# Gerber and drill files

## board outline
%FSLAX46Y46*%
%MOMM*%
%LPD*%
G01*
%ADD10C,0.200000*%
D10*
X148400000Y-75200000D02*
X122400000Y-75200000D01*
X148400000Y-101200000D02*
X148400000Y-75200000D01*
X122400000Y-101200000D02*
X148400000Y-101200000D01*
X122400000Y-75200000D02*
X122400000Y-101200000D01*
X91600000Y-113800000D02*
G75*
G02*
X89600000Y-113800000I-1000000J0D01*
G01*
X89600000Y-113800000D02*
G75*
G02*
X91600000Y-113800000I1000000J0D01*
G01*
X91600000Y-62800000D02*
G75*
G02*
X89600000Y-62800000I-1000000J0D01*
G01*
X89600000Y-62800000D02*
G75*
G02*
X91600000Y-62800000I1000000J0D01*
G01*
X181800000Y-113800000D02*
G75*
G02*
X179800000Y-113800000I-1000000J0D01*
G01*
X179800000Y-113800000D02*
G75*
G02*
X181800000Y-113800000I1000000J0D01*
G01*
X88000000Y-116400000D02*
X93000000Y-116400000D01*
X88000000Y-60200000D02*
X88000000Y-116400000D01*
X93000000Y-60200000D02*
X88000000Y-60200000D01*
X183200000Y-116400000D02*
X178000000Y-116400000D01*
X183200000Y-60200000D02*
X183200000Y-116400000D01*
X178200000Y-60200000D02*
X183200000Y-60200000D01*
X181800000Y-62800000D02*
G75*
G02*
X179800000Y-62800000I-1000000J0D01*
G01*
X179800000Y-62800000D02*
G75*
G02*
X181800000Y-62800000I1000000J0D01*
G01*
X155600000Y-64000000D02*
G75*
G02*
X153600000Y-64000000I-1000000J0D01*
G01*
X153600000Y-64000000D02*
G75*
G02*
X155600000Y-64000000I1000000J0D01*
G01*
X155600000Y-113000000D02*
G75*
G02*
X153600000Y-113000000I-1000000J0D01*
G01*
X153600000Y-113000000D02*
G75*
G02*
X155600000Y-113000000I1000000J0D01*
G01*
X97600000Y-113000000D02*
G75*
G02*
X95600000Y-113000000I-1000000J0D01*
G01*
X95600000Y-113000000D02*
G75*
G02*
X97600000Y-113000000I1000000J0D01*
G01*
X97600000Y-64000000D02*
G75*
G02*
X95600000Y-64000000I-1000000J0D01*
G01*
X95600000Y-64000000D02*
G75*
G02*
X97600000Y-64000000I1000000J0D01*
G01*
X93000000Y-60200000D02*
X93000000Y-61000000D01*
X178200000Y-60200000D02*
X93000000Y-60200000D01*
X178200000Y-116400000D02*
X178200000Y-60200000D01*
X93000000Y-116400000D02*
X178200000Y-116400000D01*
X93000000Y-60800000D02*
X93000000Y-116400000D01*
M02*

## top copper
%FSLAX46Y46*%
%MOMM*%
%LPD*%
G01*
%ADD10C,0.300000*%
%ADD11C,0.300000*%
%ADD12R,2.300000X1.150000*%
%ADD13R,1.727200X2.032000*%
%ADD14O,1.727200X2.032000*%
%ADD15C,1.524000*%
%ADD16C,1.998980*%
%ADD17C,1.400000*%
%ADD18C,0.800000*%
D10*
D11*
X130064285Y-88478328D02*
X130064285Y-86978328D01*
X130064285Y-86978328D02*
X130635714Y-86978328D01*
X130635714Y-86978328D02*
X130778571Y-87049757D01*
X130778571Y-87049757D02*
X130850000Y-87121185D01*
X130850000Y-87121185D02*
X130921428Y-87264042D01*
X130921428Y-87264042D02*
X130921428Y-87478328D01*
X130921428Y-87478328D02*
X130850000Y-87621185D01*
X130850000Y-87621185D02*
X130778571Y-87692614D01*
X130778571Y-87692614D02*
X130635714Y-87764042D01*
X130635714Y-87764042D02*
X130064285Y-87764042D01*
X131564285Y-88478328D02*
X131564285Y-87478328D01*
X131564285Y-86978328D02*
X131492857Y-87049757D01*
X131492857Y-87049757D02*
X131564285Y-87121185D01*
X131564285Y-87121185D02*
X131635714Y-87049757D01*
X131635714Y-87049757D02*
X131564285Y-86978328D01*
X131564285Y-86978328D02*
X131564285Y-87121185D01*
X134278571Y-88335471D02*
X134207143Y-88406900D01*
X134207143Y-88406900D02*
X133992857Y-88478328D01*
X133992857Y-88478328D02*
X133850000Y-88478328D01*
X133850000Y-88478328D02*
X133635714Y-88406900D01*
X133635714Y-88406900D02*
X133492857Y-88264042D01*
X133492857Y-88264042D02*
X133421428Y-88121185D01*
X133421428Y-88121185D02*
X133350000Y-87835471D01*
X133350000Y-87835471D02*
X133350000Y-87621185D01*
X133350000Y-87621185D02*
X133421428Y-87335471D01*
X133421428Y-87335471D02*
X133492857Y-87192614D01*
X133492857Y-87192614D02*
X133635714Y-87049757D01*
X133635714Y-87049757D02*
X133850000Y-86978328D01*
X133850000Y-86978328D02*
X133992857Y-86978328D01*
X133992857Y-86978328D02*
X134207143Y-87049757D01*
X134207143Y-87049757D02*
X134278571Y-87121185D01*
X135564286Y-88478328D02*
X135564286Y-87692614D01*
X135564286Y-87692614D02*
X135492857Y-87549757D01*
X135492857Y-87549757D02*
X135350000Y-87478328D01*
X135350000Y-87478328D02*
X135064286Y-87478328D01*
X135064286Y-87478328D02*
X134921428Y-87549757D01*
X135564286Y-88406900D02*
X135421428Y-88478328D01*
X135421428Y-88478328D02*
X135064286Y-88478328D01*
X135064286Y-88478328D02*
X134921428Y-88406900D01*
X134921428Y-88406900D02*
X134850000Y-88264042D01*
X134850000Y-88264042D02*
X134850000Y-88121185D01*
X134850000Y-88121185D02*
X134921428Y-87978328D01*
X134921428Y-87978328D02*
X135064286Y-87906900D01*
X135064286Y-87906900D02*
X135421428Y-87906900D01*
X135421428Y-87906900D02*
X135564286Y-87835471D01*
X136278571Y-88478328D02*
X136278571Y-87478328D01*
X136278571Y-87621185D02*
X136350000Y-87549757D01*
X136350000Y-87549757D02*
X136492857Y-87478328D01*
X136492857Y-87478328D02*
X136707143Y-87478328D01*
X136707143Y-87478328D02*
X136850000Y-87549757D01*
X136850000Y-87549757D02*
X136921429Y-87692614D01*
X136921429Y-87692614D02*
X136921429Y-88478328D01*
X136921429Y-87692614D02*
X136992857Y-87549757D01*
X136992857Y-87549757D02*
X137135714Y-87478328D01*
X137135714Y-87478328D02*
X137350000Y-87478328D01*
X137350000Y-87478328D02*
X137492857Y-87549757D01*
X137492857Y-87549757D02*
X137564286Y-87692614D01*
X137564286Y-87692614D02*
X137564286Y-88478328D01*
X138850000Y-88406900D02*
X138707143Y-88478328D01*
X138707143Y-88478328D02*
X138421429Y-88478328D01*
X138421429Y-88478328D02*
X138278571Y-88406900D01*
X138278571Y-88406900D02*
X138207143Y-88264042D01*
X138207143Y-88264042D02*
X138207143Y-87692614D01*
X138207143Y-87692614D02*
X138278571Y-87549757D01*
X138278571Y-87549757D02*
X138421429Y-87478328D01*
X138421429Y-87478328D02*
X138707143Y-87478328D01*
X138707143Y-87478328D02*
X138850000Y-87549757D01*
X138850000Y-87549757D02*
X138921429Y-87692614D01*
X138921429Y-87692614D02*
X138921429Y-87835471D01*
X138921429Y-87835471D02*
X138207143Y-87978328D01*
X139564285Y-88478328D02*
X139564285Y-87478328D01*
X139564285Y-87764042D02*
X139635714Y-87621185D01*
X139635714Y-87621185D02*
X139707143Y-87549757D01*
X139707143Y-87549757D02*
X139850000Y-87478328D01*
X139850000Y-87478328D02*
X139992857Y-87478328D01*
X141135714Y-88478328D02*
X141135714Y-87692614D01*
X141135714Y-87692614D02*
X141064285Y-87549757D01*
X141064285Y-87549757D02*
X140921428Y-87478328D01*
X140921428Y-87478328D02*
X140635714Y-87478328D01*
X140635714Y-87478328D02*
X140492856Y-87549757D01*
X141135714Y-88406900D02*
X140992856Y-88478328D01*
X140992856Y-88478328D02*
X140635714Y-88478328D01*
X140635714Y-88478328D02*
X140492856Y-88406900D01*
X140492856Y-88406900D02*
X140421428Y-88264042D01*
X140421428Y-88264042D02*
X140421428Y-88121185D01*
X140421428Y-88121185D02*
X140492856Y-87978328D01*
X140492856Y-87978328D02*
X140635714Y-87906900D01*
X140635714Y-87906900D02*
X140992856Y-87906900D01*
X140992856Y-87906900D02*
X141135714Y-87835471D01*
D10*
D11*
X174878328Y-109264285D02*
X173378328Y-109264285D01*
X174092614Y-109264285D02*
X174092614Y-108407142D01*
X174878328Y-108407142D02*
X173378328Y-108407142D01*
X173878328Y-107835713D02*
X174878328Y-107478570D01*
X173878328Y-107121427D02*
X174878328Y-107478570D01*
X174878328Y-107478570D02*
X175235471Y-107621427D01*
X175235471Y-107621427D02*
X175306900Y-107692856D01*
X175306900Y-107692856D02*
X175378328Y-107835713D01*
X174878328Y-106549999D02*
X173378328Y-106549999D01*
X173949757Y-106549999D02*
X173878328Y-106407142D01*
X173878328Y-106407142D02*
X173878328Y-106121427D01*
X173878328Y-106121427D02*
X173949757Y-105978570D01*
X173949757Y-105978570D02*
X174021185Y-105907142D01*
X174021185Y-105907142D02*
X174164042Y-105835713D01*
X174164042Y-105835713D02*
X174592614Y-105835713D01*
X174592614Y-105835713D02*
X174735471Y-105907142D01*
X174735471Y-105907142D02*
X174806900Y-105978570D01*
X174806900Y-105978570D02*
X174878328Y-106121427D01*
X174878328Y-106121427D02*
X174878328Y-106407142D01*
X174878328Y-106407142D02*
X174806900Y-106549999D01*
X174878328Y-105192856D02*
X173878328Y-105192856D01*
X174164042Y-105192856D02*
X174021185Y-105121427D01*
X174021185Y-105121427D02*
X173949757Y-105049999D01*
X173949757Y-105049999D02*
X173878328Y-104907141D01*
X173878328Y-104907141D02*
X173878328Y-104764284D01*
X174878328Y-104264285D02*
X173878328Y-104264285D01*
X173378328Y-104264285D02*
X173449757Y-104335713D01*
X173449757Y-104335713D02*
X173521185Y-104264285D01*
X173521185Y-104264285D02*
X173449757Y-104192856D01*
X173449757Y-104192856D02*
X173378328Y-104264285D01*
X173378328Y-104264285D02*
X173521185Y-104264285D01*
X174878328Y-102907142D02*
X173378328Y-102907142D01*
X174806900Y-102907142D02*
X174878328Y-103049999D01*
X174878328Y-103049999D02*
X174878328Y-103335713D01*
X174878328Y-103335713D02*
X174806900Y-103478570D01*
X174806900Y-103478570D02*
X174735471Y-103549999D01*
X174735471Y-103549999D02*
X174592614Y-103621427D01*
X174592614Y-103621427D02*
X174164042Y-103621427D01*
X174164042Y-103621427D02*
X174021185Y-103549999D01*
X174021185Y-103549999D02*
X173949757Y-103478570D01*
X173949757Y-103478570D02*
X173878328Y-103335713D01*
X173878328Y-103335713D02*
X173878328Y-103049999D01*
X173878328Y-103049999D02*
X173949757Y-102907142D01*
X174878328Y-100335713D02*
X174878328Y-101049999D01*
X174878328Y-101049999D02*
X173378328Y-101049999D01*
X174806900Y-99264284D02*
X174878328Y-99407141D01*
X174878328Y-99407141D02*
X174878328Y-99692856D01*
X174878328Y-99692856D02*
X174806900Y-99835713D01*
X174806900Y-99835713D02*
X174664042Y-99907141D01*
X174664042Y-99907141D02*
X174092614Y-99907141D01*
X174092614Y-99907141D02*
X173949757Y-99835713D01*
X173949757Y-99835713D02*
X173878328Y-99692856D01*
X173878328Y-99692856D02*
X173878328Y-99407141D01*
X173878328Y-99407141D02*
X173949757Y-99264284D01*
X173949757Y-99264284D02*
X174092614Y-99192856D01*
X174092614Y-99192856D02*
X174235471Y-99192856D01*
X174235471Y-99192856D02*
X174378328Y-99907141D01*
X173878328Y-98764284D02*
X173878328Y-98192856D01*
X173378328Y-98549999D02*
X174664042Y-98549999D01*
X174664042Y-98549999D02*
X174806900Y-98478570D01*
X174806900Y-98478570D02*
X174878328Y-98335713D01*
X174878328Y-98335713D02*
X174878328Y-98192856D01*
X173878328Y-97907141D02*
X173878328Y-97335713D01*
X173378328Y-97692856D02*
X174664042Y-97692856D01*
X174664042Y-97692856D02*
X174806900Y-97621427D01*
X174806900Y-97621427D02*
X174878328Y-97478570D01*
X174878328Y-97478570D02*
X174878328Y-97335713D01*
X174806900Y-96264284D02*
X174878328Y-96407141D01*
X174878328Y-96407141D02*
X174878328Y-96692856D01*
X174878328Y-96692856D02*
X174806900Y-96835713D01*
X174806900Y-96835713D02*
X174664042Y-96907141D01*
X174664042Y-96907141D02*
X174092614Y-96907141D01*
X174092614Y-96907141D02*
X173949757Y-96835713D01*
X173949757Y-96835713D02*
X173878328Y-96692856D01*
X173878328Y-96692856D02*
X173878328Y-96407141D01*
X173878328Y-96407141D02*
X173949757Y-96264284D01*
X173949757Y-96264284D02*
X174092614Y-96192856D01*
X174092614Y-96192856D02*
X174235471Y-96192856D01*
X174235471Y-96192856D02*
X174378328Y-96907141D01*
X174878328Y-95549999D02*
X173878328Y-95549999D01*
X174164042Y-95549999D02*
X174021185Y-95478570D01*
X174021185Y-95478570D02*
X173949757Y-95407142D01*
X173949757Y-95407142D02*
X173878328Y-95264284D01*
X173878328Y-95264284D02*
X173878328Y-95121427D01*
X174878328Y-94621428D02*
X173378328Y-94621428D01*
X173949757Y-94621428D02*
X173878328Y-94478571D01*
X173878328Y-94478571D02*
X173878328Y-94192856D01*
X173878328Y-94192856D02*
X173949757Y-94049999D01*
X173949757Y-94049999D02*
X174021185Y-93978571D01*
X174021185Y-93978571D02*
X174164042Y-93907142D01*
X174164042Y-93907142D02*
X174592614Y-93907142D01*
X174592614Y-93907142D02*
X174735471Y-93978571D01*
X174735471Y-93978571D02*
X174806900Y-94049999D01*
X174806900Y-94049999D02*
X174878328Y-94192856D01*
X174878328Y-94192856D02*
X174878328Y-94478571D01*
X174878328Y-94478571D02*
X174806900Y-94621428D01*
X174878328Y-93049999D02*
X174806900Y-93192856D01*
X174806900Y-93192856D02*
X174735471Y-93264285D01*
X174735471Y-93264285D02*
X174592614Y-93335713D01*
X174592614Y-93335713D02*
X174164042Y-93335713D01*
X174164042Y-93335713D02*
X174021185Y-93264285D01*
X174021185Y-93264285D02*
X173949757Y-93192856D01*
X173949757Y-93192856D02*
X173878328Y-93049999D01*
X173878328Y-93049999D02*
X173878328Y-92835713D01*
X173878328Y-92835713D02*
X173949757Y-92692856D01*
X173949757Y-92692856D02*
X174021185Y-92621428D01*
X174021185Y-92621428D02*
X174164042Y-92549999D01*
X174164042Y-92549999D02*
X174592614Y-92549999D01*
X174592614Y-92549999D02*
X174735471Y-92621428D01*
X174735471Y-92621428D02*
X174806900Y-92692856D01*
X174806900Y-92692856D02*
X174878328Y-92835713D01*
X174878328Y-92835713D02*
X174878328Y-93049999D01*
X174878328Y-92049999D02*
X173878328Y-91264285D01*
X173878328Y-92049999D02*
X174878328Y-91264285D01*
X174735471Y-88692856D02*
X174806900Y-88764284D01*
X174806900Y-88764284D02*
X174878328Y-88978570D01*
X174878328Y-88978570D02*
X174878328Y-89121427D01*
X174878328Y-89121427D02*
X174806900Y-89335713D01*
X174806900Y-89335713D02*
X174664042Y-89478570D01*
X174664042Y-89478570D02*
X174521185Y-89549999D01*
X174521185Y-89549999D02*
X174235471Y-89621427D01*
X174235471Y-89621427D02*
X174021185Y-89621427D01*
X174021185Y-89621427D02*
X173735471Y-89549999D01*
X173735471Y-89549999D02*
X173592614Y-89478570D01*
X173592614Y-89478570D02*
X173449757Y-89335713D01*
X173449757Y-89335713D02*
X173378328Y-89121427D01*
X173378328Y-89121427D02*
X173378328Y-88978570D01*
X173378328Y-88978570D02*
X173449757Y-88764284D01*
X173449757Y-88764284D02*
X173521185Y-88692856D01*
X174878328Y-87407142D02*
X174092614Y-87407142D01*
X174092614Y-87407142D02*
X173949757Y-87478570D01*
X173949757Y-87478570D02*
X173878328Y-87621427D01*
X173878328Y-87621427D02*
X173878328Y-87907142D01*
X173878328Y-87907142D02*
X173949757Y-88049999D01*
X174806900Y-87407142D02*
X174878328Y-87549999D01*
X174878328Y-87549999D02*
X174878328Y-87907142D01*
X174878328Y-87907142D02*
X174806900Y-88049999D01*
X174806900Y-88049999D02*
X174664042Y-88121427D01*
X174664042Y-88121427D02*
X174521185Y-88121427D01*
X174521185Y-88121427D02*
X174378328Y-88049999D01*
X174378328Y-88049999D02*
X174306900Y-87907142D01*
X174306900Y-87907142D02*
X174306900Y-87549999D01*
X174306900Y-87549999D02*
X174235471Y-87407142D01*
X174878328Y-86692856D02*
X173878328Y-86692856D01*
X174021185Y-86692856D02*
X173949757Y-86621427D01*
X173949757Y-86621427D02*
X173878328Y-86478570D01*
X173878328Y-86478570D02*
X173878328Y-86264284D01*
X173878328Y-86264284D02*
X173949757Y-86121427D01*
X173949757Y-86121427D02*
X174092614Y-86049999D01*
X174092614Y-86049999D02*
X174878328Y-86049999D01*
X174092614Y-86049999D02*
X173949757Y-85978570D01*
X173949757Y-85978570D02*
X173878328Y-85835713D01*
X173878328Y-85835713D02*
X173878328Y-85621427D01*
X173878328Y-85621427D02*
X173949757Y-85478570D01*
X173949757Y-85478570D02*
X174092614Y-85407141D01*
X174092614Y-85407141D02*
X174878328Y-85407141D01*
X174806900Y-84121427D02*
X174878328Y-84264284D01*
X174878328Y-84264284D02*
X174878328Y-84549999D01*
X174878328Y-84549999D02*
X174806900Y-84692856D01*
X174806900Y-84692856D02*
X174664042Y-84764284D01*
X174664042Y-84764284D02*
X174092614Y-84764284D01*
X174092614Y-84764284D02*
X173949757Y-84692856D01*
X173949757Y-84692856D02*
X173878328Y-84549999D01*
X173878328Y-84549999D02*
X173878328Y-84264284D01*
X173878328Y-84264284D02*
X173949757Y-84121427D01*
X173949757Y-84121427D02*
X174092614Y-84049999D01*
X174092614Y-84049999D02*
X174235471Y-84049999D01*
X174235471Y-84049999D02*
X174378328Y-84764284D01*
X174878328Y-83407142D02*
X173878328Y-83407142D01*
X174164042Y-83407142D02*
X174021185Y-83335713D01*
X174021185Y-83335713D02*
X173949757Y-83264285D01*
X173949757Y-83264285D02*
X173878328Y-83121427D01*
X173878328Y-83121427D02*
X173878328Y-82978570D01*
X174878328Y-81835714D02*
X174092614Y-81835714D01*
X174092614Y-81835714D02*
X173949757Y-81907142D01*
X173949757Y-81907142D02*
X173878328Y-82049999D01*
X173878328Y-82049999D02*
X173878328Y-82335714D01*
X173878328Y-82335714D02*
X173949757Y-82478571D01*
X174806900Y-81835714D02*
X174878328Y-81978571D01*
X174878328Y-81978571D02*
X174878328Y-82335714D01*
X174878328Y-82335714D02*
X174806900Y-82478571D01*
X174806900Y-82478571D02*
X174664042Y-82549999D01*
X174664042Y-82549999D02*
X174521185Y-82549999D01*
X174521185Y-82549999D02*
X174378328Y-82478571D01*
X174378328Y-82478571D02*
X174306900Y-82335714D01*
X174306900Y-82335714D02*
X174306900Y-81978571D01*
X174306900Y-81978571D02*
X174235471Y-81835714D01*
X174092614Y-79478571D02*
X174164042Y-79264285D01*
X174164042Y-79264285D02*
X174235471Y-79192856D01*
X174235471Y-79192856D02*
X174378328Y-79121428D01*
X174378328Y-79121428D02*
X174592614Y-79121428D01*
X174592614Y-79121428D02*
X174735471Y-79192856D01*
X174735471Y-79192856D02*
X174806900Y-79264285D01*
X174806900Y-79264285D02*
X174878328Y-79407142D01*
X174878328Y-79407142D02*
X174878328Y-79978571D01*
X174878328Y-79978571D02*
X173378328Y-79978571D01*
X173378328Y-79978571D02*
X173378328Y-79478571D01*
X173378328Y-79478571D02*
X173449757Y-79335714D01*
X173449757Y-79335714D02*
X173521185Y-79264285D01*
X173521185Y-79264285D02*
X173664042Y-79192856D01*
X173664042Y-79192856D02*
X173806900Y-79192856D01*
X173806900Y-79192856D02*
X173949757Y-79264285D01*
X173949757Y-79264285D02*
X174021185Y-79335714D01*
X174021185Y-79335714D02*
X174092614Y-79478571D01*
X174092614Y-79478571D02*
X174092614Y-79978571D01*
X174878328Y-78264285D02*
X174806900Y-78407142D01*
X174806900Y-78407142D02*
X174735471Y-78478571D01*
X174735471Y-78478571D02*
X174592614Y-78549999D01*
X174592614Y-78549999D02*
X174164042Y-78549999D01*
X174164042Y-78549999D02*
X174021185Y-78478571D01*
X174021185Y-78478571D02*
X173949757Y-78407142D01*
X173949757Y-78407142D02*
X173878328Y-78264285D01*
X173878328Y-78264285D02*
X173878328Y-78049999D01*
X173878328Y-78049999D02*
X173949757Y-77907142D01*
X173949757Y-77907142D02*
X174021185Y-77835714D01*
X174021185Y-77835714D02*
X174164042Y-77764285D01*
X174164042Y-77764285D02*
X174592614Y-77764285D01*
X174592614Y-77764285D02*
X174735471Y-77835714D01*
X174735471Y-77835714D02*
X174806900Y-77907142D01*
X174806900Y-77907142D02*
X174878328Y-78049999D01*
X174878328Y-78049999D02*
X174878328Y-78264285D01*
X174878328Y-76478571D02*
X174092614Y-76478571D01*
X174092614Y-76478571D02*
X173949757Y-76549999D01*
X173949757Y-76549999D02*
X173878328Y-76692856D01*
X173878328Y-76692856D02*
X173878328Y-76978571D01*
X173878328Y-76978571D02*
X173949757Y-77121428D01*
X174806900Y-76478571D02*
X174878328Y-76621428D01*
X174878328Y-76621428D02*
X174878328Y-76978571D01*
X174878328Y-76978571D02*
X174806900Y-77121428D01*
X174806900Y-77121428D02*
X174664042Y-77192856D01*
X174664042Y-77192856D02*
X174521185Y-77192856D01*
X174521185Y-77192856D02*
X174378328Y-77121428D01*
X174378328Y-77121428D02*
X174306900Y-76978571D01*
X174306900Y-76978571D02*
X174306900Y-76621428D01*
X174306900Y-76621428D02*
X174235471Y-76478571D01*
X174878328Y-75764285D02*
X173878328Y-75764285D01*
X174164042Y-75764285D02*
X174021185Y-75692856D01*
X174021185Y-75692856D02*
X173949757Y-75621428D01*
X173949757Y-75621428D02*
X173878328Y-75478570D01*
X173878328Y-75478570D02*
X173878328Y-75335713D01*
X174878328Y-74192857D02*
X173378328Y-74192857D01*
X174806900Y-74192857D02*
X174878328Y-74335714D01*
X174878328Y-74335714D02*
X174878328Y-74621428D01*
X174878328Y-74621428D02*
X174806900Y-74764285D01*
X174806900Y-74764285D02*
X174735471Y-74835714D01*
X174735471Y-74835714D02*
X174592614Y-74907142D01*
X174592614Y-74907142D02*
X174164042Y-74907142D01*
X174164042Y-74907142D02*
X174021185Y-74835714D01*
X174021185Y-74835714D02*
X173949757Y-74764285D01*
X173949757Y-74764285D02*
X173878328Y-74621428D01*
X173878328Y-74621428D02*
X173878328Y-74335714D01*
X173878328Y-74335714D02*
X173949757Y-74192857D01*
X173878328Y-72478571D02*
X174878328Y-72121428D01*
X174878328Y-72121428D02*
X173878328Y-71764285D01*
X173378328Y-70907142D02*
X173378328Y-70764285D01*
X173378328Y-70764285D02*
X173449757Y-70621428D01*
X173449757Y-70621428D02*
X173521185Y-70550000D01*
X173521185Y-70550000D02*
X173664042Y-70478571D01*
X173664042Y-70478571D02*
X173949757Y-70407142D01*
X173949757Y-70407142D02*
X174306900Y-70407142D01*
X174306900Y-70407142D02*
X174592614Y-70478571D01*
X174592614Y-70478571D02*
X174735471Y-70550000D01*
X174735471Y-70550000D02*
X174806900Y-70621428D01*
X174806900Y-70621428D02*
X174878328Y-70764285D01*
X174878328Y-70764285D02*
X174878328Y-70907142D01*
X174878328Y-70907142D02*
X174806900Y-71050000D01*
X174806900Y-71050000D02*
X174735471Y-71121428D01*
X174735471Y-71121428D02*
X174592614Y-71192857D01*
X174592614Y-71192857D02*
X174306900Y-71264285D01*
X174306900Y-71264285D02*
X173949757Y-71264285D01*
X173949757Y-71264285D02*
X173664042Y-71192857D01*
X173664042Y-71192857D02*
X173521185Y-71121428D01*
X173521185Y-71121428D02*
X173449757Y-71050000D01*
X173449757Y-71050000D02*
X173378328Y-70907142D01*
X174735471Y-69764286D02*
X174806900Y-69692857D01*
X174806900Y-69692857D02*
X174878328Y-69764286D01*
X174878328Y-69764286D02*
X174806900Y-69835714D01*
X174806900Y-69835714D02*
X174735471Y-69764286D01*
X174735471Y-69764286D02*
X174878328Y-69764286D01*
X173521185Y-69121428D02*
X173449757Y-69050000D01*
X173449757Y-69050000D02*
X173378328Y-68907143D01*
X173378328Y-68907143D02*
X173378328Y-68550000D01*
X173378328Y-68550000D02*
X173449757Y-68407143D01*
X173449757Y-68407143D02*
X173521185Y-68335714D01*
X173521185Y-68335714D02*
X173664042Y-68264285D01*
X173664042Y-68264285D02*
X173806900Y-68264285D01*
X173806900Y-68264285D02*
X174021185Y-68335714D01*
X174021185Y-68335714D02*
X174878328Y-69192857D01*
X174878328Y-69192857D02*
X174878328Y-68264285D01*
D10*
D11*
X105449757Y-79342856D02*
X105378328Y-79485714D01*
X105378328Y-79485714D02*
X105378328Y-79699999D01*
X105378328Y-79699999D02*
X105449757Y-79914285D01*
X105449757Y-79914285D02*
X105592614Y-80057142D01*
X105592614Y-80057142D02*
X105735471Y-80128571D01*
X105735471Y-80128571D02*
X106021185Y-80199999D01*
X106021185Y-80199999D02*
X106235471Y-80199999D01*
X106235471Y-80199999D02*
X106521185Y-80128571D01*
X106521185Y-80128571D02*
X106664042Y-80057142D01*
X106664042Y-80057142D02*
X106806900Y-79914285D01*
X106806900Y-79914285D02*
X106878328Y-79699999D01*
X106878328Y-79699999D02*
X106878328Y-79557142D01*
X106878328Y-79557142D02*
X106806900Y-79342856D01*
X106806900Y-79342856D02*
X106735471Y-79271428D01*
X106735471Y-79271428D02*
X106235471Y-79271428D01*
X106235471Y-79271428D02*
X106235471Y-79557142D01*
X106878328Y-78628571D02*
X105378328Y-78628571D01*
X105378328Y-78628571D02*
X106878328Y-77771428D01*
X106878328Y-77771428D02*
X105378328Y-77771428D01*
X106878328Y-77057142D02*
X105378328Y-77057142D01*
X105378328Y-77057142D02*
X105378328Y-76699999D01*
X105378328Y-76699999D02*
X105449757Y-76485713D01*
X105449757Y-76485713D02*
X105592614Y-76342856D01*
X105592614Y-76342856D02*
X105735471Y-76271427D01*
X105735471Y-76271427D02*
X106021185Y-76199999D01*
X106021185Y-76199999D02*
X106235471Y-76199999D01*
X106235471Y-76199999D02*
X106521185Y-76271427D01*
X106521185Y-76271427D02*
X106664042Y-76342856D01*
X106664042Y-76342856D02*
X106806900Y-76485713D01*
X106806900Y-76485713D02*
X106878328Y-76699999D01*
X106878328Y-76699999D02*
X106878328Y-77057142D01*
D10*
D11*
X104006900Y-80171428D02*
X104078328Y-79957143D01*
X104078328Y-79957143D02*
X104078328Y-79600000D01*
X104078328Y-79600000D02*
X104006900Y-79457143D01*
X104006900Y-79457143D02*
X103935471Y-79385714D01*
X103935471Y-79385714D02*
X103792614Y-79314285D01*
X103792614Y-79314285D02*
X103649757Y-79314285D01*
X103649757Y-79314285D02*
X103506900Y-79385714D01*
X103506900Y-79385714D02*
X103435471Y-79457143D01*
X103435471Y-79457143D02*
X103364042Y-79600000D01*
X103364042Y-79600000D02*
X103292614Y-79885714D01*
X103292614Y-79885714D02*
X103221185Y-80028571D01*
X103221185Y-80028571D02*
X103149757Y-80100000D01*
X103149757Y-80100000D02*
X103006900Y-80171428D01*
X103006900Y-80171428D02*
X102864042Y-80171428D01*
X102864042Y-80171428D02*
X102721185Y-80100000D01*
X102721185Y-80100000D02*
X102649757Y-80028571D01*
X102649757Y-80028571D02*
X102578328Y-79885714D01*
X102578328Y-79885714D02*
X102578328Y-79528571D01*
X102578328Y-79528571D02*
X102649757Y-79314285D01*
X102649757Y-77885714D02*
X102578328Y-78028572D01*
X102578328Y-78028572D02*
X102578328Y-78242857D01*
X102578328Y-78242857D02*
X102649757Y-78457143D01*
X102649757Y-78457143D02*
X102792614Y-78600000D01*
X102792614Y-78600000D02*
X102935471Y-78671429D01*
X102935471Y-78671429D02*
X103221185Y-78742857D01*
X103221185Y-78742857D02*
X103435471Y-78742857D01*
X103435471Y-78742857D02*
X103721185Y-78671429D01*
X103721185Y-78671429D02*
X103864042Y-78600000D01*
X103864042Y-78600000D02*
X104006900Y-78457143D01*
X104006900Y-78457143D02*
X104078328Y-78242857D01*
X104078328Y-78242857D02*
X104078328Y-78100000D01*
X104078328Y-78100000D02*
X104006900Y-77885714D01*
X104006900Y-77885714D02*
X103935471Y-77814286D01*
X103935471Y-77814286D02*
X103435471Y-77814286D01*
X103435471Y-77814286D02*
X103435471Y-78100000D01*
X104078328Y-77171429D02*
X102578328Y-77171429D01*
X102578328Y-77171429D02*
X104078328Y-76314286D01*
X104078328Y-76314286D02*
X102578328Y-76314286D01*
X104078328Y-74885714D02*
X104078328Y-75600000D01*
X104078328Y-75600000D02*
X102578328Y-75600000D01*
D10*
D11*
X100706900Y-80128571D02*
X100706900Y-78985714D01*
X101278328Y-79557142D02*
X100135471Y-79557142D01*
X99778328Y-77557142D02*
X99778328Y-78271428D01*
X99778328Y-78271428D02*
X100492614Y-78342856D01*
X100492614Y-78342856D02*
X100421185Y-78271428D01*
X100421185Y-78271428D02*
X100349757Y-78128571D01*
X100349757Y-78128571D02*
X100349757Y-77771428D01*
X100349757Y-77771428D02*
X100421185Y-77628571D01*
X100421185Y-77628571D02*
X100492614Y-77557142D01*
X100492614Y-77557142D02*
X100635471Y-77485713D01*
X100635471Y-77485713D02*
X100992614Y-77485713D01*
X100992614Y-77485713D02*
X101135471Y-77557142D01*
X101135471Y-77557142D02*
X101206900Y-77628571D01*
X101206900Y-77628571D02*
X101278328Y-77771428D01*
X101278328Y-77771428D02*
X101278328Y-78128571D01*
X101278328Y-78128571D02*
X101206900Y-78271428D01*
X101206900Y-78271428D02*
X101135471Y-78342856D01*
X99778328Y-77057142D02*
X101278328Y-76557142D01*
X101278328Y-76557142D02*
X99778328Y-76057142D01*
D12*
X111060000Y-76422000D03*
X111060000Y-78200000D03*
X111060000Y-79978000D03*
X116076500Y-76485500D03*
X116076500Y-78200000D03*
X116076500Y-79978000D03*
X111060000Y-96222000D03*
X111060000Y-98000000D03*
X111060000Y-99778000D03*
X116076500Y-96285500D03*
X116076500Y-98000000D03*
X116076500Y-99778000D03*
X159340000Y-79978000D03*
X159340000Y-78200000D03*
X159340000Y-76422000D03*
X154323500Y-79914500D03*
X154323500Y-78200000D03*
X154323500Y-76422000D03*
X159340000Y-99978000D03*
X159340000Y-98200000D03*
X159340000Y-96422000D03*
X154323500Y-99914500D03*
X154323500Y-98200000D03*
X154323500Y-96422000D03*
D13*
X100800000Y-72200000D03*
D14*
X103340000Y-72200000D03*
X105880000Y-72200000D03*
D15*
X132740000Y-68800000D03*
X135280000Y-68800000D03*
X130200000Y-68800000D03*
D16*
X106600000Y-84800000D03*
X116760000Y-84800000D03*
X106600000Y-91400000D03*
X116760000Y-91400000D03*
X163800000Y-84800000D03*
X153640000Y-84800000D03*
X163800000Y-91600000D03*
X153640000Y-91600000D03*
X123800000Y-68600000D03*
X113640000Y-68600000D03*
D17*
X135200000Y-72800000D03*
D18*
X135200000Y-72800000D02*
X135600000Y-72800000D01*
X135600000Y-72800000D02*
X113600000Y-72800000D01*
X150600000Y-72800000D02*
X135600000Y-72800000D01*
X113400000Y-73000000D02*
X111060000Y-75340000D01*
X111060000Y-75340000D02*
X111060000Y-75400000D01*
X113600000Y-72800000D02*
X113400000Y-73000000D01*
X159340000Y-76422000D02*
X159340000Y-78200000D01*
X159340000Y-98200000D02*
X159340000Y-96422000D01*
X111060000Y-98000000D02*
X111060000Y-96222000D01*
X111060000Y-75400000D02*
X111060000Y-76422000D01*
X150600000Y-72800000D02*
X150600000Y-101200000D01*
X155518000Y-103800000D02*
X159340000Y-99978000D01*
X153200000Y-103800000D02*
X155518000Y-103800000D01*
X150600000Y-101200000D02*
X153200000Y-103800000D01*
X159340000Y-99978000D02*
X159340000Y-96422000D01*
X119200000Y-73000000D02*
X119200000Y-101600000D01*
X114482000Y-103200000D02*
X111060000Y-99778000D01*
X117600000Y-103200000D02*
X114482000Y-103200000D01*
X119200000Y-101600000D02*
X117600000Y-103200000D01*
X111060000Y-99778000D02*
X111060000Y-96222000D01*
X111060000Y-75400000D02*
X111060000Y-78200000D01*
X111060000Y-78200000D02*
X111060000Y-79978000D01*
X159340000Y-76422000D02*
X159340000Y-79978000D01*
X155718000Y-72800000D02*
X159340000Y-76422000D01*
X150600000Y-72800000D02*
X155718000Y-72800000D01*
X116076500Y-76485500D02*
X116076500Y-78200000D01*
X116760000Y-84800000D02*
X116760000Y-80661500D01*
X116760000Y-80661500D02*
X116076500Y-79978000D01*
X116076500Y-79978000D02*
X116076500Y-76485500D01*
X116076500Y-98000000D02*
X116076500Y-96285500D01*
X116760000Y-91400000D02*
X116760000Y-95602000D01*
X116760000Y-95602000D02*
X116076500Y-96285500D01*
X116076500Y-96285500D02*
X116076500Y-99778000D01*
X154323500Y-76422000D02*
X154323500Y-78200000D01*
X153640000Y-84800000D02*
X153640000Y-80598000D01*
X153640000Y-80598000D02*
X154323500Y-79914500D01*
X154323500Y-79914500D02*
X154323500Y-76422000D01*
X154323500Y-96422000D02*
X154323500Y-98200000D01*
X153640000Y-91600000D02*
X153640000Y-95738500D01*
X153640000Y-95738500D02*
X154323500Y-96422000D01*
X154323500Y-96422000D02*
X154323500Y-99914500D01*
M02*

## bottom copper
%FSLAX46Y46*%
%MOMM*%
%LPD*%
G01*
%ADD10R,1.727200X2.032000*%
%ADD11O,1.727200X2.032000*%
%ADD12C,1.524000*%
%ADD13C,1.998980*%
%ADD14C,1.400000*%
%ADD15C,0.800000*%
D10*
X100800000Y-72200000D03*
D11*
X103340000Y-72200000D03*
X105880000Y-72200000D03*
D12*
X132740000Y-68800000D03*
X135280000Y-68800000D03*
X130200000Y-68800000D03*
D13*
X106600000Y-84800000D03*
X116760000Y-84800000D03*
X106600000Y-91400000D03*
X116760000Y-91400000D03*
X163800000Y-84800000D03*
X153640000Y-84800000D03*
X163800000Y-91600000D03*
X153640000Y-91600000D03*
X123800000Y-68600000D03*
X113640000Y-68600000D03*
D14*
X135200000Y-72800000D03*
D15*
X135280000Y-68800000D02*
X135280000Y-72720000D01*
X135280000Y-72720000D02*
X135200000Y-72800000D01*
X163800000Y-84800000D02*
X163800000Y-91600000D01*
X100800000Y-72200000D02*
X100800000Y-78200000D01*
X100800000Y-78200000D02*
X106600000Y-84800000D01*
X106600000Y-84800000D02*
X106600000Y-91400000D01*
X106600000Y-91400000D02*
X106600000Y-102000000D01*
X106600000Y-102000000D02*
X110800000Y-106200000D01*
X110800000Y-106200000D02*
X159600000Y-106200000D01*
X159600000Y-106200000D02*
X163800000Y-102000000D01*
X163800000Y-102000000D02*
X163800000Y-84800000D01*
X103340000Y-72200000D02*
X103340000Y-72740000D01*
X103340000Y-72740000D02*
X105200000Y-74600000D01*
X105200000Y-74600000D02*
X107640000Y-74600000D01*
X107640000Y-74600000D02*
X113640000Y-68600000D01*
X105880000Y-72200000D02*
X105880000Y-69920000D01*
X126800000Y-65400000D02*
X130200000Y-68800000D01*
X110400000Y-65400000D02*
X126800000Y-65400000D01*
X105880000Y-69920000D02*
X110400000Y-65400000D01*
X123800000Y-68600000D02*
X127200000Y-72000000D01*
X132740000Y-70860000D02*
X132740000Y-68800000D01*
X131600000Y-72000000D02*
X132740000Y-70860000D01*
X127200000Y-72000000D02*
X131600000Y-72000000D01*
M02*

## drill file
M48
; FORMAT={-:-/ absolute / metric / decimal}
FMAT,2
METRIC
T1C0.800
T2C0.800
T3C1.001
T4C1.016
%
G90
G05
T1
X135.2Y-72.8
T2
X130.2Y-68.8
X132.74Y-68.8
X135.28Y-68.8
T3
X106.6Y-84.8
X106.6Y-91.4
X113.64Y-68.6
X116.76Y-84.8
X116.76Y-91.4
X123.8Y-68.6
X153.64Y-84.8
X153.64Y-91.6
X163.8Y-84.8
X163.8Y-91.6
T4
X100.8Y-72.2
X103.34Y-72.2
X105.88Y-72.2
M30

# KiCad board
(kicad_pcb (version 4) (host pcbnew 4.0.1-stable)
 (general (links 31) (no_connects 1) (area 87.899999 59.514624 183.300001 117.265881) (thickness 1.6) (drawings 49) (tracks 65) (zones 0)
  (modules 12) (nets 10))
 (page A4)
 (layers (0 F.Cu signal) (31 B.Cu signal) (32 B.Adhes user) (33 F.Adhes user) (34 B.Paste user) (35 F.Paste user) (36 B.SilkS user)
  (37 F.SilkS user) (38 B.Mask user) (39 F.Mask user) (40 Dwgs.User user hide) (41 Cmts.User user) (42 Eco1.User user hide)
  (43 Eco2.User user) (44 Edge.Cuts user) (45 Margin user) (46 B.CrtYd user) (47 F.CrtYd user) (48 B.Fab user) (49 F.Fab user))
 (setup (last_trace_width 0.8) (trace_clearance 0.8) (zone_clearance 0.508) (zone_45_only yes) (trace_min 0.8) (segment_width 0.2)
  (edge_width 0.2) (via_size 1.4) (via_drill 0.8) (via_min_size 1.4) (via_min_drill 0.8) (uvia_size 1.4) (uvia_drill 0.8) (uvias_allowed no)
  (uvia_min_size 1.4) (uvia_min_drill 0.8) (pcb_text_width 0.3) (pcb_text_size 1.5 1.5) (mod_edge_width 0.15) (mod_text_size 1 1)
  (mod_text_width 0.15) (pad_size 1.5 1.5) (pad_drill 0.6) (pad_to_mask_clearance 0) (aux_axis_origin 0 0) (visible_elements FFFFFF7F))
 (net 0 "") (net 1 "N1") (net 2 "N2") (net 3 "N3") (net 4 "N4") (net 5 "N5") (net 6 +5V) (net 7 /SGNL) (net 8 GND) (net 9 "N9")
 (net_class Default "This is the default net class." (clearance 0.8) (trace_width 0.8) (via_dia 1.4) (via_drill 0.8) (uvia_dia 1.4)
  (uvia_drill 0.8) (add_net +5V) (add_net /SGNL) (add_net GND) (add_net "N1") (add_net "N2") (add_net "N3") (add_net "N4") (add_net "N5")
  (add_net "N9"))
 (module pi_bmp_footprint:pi (layer F.Cu) (at 135.4 88.2)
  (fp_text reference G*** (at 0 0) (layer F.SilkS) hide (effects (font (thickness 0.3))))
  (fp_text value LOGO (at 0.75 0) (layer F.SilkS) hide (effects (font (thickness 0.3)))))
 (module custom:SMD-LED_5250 (layer F.Cu) (at 113.6 78.2)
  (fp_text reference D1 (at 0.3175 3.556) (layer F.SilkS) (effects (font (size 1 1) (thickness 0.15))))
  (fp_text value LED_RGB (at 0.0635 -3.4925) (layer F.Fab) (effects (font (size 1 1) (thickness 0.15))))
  (pad 1 smd rect (at -2.54 -1.778) (size 2.3 1.15) (layers F.Cu F.Paste F.Mask) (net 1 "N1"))
  (pad 2 smd rect (at -2.54 0) (size 2.3 1.15) (layers F.Cu F.Paste F.Mask) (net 1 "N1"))
  (pad 3 smd rect (at -2.54 1.778) (size 2.3 1.15) (layers F.Cu F.Paste F.Mask) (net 1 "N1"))
  (pad 4 smd rect (at 2.4765 -1.7145) (size 2.3 1.15) (layers F.Cu F.Paste F.Mask) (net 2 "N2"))
  (pad 5 smd rect (at 2.4765 0) (size 2.3 1.15) (layers F.Cu F.Paste F.Mask) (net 2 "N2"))
  (pad 6 smd rect (at 2.4765 1.778) (size 2.3 1.15) (layers F.Cu F.Paste F.Mask) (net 2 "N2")))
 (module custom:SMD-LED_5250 (layer F.Cu) (at 113.6 98)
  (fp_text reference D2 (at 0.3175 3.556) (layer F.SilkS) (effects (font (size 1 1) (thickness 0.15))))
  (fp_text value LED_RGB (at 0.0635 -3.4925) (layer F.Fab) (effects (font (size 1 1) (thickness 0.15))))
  (pad 1 smd rect (at -2.54 -1.778) (size 2.3 1.15) (layers F.Cu F.Paste F.Mask) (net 1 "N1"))
  (pad 2 smd rect (at -2.54 0) (size 2.3 1.15) (layers F.Cu F.Paste F.Mask) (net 1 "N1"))
  (pad 3 smd rect (at -2.54 1.778) (size 2.3 1.15) (layers F.Cu F.Paste F.Mask) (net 1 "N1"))
  (pad 4 smd rect (at 2.4765 -1.7145) (size 2.3 1.15) (layers F.Cu F.Paste F.Mask) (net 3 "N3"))
  (pad 5 smd rect (at 2.4765 0) (size 2.3 1.15) (layers F.Cu F.Paste F.Mask) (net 3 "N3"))
  (pad 6 smd rect (at 2.4765 1.778) (size 2.3 1.15) (layers F.Cu F.Paste F.Mask) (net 3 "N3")))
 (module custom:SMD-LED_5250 (layer F.Cu) (at 156.8 78.2 180)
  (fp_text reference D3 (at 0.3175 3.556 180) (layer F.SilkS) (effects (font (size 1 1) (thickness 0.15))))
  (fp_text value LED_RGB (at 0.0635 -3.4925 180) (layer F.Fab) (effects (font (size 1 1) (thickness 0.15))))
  (pad 1 smd rect (at -2.54 -1.778 180) (size 2.3 1.15) (layers F.Cu F.Paste F.Mask) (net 1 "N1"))
  (pad 2 smd rect (at -2.54 0 180) (size 2.3 1.15) (layers F.Cu F.Paste F.Mask) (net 1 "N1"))
  (pad 3 smd rect (at -2.54 1.778 180) (size 2.3 1.15) (layers F.Cu F.Paste F.Mask) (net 1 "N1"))
  (pad 4 smd rect (at 2.4765 -1.7145 180) (size 2.3 1.15) (layers F.Cu F.Paste F.Mask) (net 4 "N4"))
  (pad 5 smd rect (at 2.4765 0 180) (size 2.3 1.15) (layers F.Cu F.Paste F.Mask) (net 4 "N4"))
  (pad 6 smd rect (at 2.4765 1.778 180) (size 2.3 1.15) (layers F.Cu F.Paste F.Mask) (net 4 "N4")))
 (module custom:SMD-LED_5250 (layer F.Cu) (at 156.8 98.2 180)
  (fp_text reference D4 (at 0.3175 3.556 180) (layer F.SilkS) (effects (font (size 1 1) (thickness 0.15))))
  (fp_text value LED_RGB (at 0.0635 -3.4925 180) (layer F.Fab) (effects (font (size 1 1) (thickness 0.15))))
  (pad 1 smd rect (at -2.54 -1.778 180) (size 2.3 1.15) (layers F.Cu F.Paste F.Mask) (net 1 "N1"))
  (pad 2 smd rect (at -2.54 0 180) (size 2.3 1.15) (layers F.Cu F.Paste F.Mask) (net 1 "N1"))
  (pad 3 smd rect (at -2.54 1.778 180) (size 2.3 1.15) (layers F.Cu F.Paste F.Mask) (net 1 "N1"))
  (pad 4 smd rect (at 2.4765 -1.7145 180) (size 2.3 1.15) (layers F.Cu F.Paste F.Mask) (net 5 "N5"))
  (pad 5 smd rect (at 2.4765 0 180) (size 2.3 1.15) (layers F.Cu F.Paste F.Mask) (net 5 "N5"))
  (pad 6 smd rect (at 2.4765 1.778 180) (size 2.3 1.15) (layers F.Cu F.Paste F.Mask) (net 5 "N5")))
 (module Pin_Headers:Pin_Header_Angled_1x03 (layer F.Cu) (at 100.8 72.2 90)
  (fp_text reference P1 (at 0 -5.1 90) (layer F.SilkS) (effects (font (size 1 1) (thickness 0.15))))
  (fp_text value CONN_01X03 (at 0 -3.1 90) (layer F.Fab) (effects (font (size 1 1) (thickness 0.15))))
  (pad 1 thru_hole rect (at 0 0 90) (size 2.032 1.7272) (drill 1.016) (layers *.Cu *.Mask F.SilkS) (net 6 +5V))
  (pad 2 thru_hole oval (at 0 2.54 90) (size 2.032 1.7272) (drill 1.016) (layers *.Cu *.Mask F.SilkS) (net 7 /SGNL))
  (pad 3 thru_hole oval (at 0 5.08 90) (size 2.032 1.7272) (drill 1.016) (layers *.Cu *.Mask F.SilkS) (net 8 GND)))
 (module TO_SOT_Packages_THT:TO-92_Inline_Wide (layer F.Cu) (at 130.2 68.8)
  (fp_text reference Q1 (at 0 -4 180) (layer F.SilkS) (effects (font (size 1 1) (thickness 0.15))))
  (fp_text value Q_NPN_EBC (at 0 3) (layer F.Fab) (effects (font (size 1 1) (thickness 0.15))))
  (pad 2 thru_hole circle (at 2.54 0 90) (size 1.524 1.524) (drill 0.8) (layers *.Cu *.Mask F.SilkS) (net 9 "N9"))
  (pad 3 thru_hole circle (at 5.08 0 90) (size 1.524 1.524) (drill 0.8) (layers *.Cu *.Mask F.SilkS) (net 1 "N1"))
  (pad 1 thru_hole circle (at 0 0 90) (size 1.524 1.524) (drill 0.8) (layers *.Cu *.Mask F.SilkS) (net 8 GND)))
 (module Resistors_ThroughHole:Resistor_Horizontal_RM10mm (layer F.Cu) (at 106.6 84.8)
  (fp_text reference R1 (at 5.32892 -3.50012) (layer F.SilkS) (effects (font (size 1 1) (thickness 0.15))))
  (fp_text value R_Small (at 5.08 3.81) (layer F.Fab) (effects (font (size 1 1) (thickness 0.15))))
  (pad 1 thru_hole circle (at 0 0) (size 1.99898 1.99898) (drill 1.00076) (layers *.Cu *.SilkS *.Mask) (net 6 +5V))
  (pad 2 thru_hole circle (at 10.16 0) (size 1.99898 1.99898) (drill 1.00076) (layers *.Cu *.SilkS *.Mask) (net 2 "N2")))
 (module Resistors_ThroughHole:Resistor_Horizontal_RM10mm (layer F.Cu) (at 106.6 91.4)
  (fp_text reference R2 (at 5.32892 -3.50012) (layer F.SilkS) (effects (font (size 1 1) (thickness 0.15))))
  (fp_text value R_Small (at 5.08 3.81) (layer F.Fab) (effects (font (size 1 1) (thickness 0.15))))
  (pad 1 thru_hole circle (at 0 0) (size 1.99898 1.99898) (drill 1.00076) (layers *.Cu *.SilkS *.Mask) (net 6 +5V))
  (pad 2 thru_hole circle (at 10.16 0) (size 1.99898 1.99898) (drill 1.00076) (layers *.Cu *.SilkS *.Mask) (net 3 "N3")))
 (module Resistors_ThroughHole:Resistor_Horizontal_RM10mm (layer F.Cu) (at 163.8 84.8 180)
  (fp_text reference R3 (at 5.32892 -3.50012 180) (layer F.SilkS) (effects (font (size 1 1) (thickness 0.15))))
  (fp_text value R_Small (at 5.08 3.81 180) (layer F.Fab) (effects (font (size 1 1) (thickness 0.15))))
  (pad 1 thru_hole circle (at 0 0 180) (size 1.99898 1.99898) (drill 1.00076) (layers *.Cu *.SilkS *.Mask) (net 6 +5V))
  (pad 2 thru_hole circle (at 10.16 0 180) (size 1.99898 1.99898) (drill 1.00076) (layers *.Cu *.SilkS *.Mask) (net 4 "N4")))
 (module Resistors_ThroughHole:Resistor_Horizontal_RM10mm (layer F.Cu) (at 163.8 91.6 180)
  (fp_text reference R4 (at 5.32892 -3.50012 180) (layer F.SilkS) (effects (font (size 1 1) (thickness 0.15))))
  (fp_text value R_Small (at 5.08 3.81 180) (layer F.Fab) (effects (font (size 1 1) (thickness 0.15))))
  (pad 1 thru_hole circle (at 0 0 180) (size 1.99898 1.99898) (drill 1.00076) (layers *.Cu *.SilkS *.Mask) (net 6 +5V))
  (pad 2 thru_hole circle (at 10.16 0 180) (size 1.99898 1.99898) (drill 1.00076) (layers *.Cu *.SilkS *.Mask) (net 5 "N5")))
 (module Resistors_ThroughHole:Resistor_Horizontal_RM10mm (layer F.Cu) (at 123.8 68.6 180)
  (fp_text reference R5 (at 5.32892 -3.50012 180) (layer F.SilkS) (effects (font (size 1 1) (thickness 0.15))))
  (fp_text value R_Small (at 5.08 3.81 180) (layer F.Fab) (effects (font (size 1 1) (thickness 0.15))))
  (pad 1 thru_hole circle (at 0 0 180) (size 1.99898 1.99898) (drill 1.00076) (layers *.Cu *.SilkS *.Mask) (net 9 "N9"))
  (pad 2 thru_hole circle (at 10.16 0 180) (size 1.99898 1.99898) (drill 1.00076) (layers *.Cu *.SilkS *.Mask) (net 7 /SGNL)))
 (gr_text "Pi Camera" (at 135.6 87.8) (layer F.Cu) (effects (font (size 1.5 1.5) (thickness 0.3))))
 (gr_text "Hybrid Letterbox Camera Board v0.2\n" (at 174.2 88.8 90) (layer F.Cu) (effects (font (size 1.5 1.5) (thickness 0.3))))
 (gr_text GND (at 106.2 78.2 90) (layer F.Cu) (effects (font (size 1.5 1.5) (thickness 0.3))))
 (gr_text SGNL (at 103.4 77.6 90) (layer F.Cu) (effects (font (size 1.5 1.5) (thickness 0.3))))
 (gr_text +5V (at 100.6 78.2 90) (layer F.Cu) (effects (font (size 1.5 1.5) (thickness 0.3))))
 (gr_line (start 148.4 75.2) (end 122.4 75.2) (angle 90) (layer Edge.Cuts) (width 0.2))
 (gr_line (start 148.4 101.2) (end 148.4 75.2) (angle 90) (layer Edge.Cuts) (width 0.2))
 (gr_line (start 122.4 101.2) (end 148.4 101.2) (angle 90) (layer Edge.Cuts) (width 0.2))
 (gr_line (start 122.4 75.2) (end 122.4 101.2) (angle 90) (layer Edge.Cuts) (width 0.2))
 (gr_circle (center 90.6 113.8) (end 91.4 114.4) (layer Edge.Cuts) (width 0.2))
 (gr_circle (center 90.6 62.8) (end 91.4 63.4) (layer Edge.Cuts) (width 0.2))
 (gr_circle (center 180.8 113.8) (end 181.6 114.4) (layer Edge.Cuts) (width 0.2))
 (gr_line (start 88 116.4) (end 93 116.4) (angle 90) (layer Edge.Cuts) (width 0.2))
 (gr_line (start 88 60.2) (end 88 116.4) (angle 90) (layer Edge.Cuts) (width 0.2))
 (gr_line (start 93 60.2) (end 88 60.2) (angle 90) (layer Edge.Cuts) (width 0.2))
 (gr_line (start 183.2 116.4) (end 178 116.4) (angle 90) (layer Edge.Cuts) (width 0.2))
 (gr_line (start 183.2 60.2) (end 183.2 116.4) (angle 90) (layer Edge.Cuts) (width 0.2))
 (gr_line (start 178.2 60.2) (end 183.2 60.2) (angle 90) (layer Edge.Cuts) (width 0.2))
 (gr_circle (center 180.8 62.8) (end 181.6 63.4) (layer Edge.Cuts) (width 0.2))
 (gr_circle (center 154.6 64) (end 155.4 64.6) (layer Edge.Cuts) (width 0.2))
 (gr_circle (center 154.6 113) (end 155.4 113.6) (layer Edge.Cuts) (width 0.2))
 (gr_circle (center 96.6 113) (end 97.4 113.6) (layer Edge.Cuts) (width 0.2))
 (gr_circle (center 96.6 64) (end 97.4 64.6) (layer Edge.Cuts) (width 0.2))
 (gr_line (start 93 60.2) (end 93 61) (angle 90) (layer Edge.Cuts) (width 0.2))
 (gr_line (start 178.2 60.2) (end 93 60.2) (angle 90) (layer Edge.Cuts) (width 0.2))
 (gr_line (start 178.2 116.4) (end 178.2 60.2) (angle 90) (layer Edge.Cuts) (width 0.2))
 (gr_line (start 93 116.4) (end 178.2 116.4) (angle 90) (layer Edge.Cuts) (width 0.2))
 (gr_line (start 93 60.8) (end 93 116.4) (angle 90) (layer Edge.Cuts) (width 0.2))
 (segment (start 135.28 68.8) (end 135.28 72.72) (width 0.8) (layer B.Cu) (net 1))
 (segment (start 135.2 72.8) (end 135.6 72.8) (width 0.8) (layer F.Cu) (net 1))
 (via (at 135.2 72.8) (size 1.4) (drill 0.8) (layers F.Cu B.Cu) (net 1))
 (segment (start 135.28 72.72) (end 135.2 72.8) (width 0.8) (layer B.Cu) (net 1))
 (segment (start 135.6 72.8) (end 113.6 72.8) (width 0.8) (layer F.Cu) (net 1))
 (segment (start 150.6 72.8) (end 135.6 72.8) (width 0.8) (layer F.Cu) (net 1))
 (segment (start 113.4 73) (end 111.06 75.34) (width 0.8) (layer F.Cu) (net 1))
 (segment (start 111.06 75.34) (end 111.06 75.4) (width 0.8) (layer F.Cu) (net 1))
 (segment (start 113.6 72.8) (end 113.4 73) (width 0.8) (layer F.Cu) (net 1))
 (segment (start 159.34 76.422) (end 159.34 78.2) (width 0.8) (layer F.Cu) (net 1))
 (segment (start 159.34 98.2) (end 159.34 96.422) (width 0.8) (layer F.Cu) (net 1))
 (segment (start 111.06 98) (end 111.06 96.222) (width 0.8) (layer F.Cu) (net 1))
 (segment (start 111.06 75.4) (end 111.06 76.422) (width 0.8) (layer F.Cu) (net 1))
 (segment (start 150.6 72.8) (end 150.6 101.2) (width 0.8) (layer F.Cu) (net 1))
 (segment (start 155.518 103.8) (end 159.34 99.978) (width 0.8) (layer F.Cu) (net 1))
 (segment (start 153.2 103.8) (end 155.518 103.8) (width 0.8) (layer F.Cu) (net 1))
 (segment (start 150.6 101.2) (end 153.2 103.8) (width 0.8) (layer F.Cu) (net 1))
 (segment (start 159.34 99.978) (end 159.34 96.422) (width 0.8) (layer F.Cu) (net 1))
 (segment (start 119.2 73) (end 119.2 101.6) (width 0.8) (layer F.Cu) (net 1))
 (segment (start 114.482 103.2) (end 111.06 99.778) (width 0.8) (layer F.Cu) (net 1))
 (segment (start 117.6 103.2) (end 114.482 103.2) (width 0.8) (layer F.Cu) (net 1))
 (segment (start 119.2 101.6) (end 117.6 103.2) (width 0.8) (layer F.Cu) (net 1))
 (segment (start 111.06 99.778) (end 111.06 96.222) (width 0.8) (layer F.Cu) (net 1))
 (segment (start 111.06 75.4) (end 111.06 78.2) (width 0.8) (layer F.Cu) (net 1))
 (segment (start 111.06 78.2) (end 111.06 79.978) (width 0.8) (layer F.Cu) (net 1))
 (segment (start 159.34 76.422) (end 159.34 79.978) (width 0.8) (layer F.Cu) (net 1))
 (segment (start 155.718 72.8) (end 159.34 76.422) (width 0.8) (layer F.Cu) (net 1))
 (segment (start 150.6 72.8) (end 155.718 72.8) (width 0.8) (layer F.Cu) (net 1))
 (segment (start 116.0765 76.4855) (end 116.0765 78.2) (width 0.8) (layer F.Cu) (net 2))
 (segment (start 116.76 84.8) (end 116.76 80.6615) (width 0.8) (layer F.Cu) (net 2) (status 10))
 (segment (start 116.76 80.6615) (end 116.0765 79.978) (width 0.8) (layer F.Cu) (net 2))
 (segment (start 116.0765 79.978) (end 116.0765 76.4855) (width 0.8) (layer F.Cu) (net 2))
 (segment (start 116.0765 98) (end 116.0765 96.2855) (width 0.8) (layer F.Cu) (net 3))
 (segment (start 116.76 91.4) (end 116.76 95.602) (width 0.8) (layer F.Cu) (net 3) (status 10))
 (segment (start 116.76 95.602) (end 116.0765 96.2855) (width 0.8) (layer F.Cu) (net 3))
 (segment (start 116.0765 96.2855) (end 116.0765 99.778) (width 0.8) (layer F.Cu) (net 3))
 (segment (start 154.3235 76.422) (end 154.3235 78.2) (width 0.8) (layer F.Cu) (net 4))
 (segment (start 153.64 84.8) (end 153.64 80.598) (width 0.8) (layer F.Cu) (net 4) (status 10))
 (segment (start 153.64 80.598) (end 154.3235 79.9145) (width 0.8) (layer F.Cu) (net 4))
 (segment (start 154.3235 79.9145) (end 154.3235 76.422) (width 0.8) (layer F.Cu) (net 4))
 (segment (start 154.3235 96.422) (end 154.3235 98.2) (width 0.8) (layer F.Cu) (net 5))
 (segment (start 153.64 91.6) (end 153.64 95.7385) (width 0.8) (layer F.Cu) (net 5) (status 10))
 (segment (start 153.64 95.7385) (end 154.3235 96.422) (width 0.8) (layer F.Cu) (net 5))
 (segment (start 154.3235 96.422) (end 154.3235 99.9145) (width 0.8) (layer F.Cu) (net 5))
 (segment (start 163.8 84.8) (end 163.8 91.6) (width 0.8) (layer B.Cu) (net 6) (status 20))
 (segment (start 100.8 72.2) (end 100.8 78.2) (width 0.8) (layer B.Cu) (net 6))
 (segment (start 100.8 78.2) (end 106.6 84.8) (width 0.8) (layer B.Cu) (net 6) (status 20))
 (segment (start 106.6 84.8) (end 106.6 91.4) (width 0.8) (layer B.Cu) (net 6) (status 10))
 (segment (start 106.6 91.4) (end 106.6 102) (width 0.8) (layer B.Cu) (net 6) (status 10))
 (segment (start 106.6 102) (end 110.8 106.2) (width 0.8) (layer B.Cu) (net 6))
 (segment (start 110.8 106.2) (end 159.6 106.2) (width 0.8) (layer B.Cu) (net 6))
 (segment (start 159.6 106.2) (end 163.8 102) (width 0.8) (layer B.Cu) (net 6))
 (segment (start 163.8 102) (end 163.8 84.8) (width 0.8) (layer B.Cu) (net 6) (status 20))
 (segment (start 103.34 72.2) (end 103.34 72.74) (width 0.8) (layer B.Cu) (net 7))
 (segment (start 103.34 72.74) (end 105.2 74.6) (width 0.8) (layer B.Cu) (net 7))
 (segment (start 105.2 74.6) (end 107.64 74.6) (width 0.8) (layer B.Cu) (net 7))
 (segment (start 107.64 74.6) (end 113.64 68.6) (width 0.8) (layer B.Cu) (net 7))
 (segment (start 105.88 72.2) (end 105.88 69.92) (width 0.8) (layer B.Cu) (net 8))
 (segment (start 126.8 65.4) (end 130.2 68.8) (width 0.8) (layer B.Cu) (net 8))
 (segment (start 110.4 65.4) (end 126.8 65.4) (width 0.8) (layer B.Cu) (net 8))
 (segment (start 105.88 69.92) (end 110.4 65.4) (width 0.8) (layer B.Cu) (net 8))
 (segment (start 123.8 68.6) (end 127.2 72) (width 0.8) (layer B.Cu) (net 9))
 (segment (start 132.74 70.86) (end 132.74 68.8) (width 0.8) (layer B.Cu) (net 9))
 (segment (start 131.6 72) (end 132.74 70.86) (width 0.8) (layer B.Cu) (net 9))
 (segment (start 127.2 72) (end 131.6 72) (width 0.8) (layer B.Cu) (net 9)))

